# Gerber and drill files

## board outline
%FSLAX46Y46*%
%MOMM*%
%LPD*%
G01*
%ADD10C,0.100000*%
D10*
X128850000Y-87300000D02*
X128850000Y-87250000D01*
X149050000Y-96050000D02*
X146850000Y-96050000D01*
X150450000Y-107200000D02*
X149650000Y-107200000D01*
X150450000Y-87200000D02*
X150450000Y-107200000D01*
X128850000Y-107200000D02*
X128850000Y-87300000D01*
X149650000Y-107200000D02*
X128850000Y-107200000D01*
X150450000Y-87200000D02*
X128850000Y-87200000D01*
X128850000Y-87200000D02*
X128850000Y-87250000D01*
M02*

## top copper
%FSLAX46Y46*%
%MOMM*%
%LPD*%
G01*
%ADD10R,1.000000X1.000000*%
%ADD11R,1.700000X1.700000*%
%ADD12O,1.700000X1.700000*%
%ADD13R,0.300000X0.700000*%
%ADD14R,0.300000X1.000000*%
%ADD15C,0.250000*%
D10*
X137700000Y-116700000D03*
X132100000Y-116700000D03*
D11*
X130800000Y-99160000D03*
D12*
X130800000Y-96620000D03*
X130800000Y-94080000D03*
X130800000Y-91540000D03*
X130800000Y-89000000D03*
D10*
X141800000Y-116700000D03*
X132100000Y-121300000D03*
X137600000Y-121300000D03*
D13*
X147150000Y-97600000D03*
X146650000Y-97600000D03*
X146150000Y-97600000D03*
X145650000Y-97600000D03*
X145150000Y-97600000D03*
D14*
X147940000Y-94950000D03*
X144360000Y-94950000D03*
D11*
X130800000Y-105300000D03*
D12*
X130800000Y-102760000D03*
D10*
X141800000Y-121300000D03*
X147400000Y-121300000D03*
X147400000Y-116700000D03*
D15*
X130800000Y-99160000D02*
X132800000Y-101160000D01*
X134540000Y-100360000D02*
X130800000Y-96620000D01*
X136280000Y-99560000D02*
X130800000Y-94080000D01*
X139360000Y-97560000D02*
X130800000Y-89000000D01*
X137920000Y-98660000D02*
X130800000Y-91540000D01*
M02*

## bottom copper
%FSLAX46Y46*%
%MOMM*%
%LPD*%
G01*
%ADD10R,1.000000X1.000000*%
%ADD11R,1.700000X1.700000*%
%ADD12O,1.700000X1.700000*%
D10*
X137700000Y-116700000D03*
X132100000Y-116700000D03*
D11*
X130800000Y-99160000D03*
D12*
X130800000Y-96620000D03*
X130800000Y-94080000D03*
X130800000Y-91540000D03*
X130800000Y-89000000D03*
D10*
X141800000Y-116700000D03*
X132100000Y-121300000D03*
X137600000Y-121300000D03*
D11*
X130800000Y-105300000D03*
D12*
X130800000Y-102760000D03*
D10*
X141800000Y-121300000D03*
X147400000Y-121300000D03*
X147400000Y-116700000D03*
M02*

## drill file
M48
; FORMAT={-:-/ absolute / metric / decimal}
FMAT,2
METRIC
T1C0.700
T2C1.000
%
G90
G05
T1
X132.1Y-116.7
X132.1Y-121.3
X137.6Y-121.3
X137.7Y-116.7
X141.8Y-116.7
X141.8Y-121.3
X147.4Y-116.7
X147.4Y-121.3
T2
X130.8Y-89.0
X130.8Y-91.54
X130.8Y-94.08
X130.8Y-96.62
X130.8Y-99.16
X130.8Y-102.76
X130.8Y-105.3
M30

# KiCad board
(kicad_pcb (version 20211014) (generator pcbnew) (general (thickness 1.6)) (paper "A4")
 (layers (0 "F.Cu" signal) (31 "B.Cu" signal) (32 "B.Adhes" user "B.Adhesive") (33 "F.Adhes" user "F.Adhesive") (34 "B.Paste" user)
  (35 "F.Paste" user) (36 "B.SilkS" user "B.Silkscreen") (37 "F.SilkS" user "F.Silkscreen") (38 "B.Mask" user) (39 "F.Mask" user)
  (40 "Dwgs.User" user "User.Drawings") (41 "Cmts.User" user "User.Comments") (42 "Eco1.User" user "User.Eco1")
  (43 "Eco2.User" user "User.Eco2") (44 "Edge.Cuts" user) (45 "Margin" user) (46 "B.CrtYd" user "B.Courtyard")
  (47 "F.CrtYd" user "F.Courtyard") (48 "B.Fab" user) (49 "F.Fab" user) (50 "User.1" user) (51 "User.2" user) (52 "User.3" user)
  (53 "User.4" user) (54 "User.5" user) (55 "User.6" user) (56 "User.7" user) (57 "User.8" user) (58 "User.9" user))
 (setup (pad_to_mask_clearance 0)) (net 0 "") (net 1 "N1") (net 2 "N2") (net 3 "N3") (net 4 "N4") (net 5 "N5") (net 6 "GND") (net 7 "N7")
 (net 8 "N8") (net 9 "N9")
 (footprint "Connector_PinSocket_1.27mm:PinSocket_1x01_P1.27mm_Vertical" (layer "F.Cu") (at 137.7 116.7)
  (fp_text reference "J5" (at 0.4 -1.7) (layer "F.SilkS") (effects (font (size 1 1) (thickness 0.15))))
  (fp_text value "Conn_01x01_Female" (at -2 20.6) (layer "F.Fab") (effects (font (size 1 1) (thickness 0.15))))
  (pad "1" thru_hole rect (at 0 0) (size 1 1) (drill 0.7) (layers *.Cu *.Mask) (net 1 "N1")))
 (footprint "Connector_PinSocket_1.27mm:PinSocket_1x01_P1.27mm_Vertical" (layer "F.Cu") (at 132.1 116.7)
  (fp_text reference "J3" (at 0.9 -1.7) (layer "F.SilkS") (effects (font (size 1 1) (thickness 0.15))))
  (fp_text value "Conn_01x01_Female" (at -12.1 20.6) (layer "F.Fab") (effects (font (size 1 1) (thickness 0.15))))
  (pad "1" thru_hole rect (at 0 0) (size 1 1) (drill 0.7) (layers *.Cu *.Mask) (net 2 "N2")))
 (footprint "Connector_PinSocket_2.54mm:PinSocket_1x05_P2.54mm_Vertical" (layer "F.Cu") (at 130.8 99.16 180)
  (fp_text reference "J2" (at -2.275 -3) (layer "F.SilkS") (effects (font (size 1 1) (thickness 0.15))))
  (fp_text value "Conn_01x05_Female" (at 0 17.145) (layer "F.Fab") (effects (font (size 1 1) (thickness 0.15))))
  (pad "1" thru_hole rect (at 0 0 180) (size 1.7 1.7) (drill 1) (layers *.Cu *.Mask) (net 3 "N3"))
  (pad "2" thru_hole oval (at 0 2.54 180) (size 1.7 1.7) (drill 1) (layers *.Cu *.Mask) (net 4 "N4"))
  (pad "3" thru_hole oval (at 0 5.08 180) (size 1.7 1.7) (drill 1) (layers *.Cu *.Mask) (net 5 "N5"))
  (pad "4" thru_hole oval (at 0 7.62 180) (size 1.7 1.7) (drill 1) (layers *.Cu *.Mask) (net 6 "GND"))
  (pad "5" thru_hole oval (at 0 10.16 180) (size 1.7 1.7) (drill 1) (layers *.Cu *.Mask) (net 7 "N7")))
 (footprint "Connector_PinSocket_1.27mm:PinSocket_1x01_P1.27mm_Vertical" (layer "F.Cu") (at 141.8 116.7)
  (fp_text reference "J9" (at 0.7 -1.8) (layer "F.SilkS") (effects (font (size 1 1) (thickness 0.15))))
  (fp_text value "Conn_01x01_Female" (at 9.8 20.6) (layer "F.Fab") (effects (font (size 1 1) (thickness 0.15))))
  (pad "1" thru_hole rect (at 0 0) (size 1 1) (drill 0.7) (layers *.Cu *.Mask) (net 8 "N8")))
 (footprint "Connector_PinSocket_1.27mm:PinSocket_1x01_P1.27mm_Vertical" (layer "F.Cu") (at 132.1 121.3)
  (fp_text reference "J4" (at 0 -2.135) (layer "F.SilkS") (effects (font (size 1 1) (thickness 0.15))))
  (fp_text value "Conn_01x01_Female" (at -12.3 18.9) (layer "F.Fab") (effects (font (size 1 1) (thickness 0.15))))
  (pad "1" thru_hole rect (at 0 0) (size 1 1) (drill 0.7) (layers *.Cu *.Mask) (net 3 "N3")))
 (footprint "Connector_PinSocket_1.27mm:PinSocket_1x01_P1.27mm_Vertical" (layer "F.Cu") (at 137.6 121.3)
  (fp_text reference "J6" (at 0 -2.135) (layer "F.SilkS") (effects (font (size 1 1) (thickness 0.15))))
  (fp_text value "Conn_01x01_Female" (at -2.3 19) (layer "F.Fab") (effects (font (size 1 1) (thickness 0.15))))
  (pad "1" thru_hole rect (at 0 0) (size 1 1) (drill 0.7) (layers *.Cu *.Mask) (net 6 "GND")))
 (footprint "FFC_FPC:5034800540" (layer "F.Cu") (at 146.15 96.1 180)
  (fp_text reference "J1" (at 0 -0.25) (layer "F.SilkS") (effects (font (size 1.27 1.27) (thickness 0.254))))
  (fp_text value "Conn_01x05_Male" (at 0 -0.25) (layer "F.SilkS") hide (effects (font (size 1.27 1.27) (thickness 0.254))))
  (pad "1" smd rect (at -1 -1.5 180) (size 0.3 0.7) (layers "F.Cu" "F.Paste" "F.Mask") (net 3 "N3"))
  (pad "2" smd rect (at -0.5 -1.5 180) (size 0.3 0.7) (layers "F.Cu" "F.Paste" "F.Mask") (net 4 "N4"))
  (pad "3" smd rect (at 0 -1.5 180) (size 0.3 0.7) (layers "F.Cu" "F.Paste" "F.Mask") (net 5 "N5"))
  (pad "4" smd rect (at 0.5 -1.5 180) (size 0.3 0.7) (layers "F.Cu" "F.Paste" "F.Mask") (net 6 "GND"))
  (pad "5" smd rect (at 1 -1.5 180) (size 0.3 0.7) (layers "F.Cu" "F.Paste" "F.Mask") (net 7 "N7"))
  (pad "MP1" smd rect (at -1.79 1.15 180) (size 0.3 1) (layers "F.Cu" "F.Paste" "F.Mask"))
  (pad "MP2" smd rect (at 1.79 1.15 180) (size 0.3 1) (layers "F.Cu" "F.Paste" "F.Mask")))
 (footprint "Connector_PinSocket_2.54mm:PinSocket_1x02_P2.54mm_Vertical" (layer "F.Cu") (at 130.8 105.3 180)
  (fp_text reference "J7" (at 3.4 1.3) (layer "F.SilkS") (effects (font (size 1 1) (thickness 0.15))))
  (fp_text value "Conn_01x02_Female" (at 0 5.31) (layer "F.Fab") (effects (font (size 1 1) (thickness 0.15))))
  (pad "1" thru_hole rect (at 0 0 180) (size 1.7 1.7) (drill 1) (layers *.Cu *.Mask) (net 1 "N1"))
  (pad "2" thru_hole oval (at 0 2.54 180) (size 1.7 1.7) (drill 1) (layers *.Cu *.Mask) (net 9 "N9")))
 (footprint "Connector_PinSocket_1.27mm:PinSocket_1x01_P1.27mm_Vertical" (layer "F.Cu") (at 141.8 121.3)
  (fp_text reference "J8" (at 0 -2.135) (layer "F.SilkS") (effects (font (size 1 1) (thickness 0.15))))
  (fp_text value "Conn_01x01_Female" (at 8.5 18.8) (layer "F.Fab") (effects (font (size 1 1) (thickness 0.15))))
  (pad "1" thru_hole rect (at 0 0) (size 1 1) (drill 0.7) (layers *.Cu *.Mask) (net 3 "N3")))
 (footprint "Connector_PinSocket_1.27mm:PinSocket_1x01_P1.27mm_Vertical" (layer "F.Cu") (at 147.4 121.3)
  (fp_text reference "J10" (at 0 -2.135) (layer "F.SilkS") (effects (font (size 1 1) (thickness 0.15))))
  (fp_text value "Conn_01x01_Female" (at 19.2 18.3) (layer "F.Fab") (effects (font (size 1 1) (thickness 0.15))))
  (pad "1" thru_hole rect (at 0 0) (size 1 1) (drill 0.7) (layers *.Cu *.Mask) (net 6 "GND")))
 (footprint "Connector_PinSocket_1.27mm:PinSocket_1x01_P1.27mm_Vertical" (layer "F.Cu") (at 147.4 116.7)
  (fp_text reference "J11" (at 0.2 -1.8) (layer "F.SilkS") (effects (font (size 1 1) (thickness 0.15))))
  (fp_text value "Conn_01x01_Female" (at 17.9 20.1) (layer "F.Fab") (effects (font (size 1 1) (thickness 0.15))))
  (pad "1" thru_hole rect (at 0 0) (size 1 1) (drill 0.7) (layers *.Cu *.Mask) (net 9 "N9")))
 (gr_line (start 128.85 87.3) (end 128.85 87.25) (layer "Edge.Cuts") (width 0.1))
 (gr_line (start 149.05 96.05) (end 146.85 96.05) (layer "Edge.Cuts") (width 0.1))
 (gr_line (start 150.45 107.2) (end 149.65 107.2) (layer "Edge.Cuts") (width 0.1))
 (gr_line (start 150.45 87.2) (end 150.45 107.2) (layer "Edge.Cuts") (width 0.1))
 (gr_line (start 128.85 107.2) (end 128.85 87.3) (layer "Edge.Cuts") (width 0.1))
 (gr_line (start 149.65 107.2) (end 128.85 107.2) (layer "Edge.Cuts") (width 0.1))
 (gr_line (start 150.45 87.2) (end 128.85 87.2) (layer "Edge.Cuts") (width 0.1))
 (gr_line (start 128.85 87.2) (end 128.85 87.25) (layer "Edge.Cuts") (width 0.1))
 (segment (start 130.8 99.16) (end 132.8 101.16) (width 0.25) (layer "F.Cu") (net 3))
 (segment (start 134.54 100.36) (end 130.8 96.62) (width 0.25) (layer "F.Cu") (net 4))
 (segment (start 136.28 99.56) (end 130.8 94.08) (width 0.25) (layer "F.Cu") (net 5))
 (segment (start 139.36 97.56) (end 130.8 89) (width 0.25) (layer "F.Cu") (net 7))
 (segment (start 137.92 98.66) (end 130.8 91.54) (width 0.25) (layer "F.Cu") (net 6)))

